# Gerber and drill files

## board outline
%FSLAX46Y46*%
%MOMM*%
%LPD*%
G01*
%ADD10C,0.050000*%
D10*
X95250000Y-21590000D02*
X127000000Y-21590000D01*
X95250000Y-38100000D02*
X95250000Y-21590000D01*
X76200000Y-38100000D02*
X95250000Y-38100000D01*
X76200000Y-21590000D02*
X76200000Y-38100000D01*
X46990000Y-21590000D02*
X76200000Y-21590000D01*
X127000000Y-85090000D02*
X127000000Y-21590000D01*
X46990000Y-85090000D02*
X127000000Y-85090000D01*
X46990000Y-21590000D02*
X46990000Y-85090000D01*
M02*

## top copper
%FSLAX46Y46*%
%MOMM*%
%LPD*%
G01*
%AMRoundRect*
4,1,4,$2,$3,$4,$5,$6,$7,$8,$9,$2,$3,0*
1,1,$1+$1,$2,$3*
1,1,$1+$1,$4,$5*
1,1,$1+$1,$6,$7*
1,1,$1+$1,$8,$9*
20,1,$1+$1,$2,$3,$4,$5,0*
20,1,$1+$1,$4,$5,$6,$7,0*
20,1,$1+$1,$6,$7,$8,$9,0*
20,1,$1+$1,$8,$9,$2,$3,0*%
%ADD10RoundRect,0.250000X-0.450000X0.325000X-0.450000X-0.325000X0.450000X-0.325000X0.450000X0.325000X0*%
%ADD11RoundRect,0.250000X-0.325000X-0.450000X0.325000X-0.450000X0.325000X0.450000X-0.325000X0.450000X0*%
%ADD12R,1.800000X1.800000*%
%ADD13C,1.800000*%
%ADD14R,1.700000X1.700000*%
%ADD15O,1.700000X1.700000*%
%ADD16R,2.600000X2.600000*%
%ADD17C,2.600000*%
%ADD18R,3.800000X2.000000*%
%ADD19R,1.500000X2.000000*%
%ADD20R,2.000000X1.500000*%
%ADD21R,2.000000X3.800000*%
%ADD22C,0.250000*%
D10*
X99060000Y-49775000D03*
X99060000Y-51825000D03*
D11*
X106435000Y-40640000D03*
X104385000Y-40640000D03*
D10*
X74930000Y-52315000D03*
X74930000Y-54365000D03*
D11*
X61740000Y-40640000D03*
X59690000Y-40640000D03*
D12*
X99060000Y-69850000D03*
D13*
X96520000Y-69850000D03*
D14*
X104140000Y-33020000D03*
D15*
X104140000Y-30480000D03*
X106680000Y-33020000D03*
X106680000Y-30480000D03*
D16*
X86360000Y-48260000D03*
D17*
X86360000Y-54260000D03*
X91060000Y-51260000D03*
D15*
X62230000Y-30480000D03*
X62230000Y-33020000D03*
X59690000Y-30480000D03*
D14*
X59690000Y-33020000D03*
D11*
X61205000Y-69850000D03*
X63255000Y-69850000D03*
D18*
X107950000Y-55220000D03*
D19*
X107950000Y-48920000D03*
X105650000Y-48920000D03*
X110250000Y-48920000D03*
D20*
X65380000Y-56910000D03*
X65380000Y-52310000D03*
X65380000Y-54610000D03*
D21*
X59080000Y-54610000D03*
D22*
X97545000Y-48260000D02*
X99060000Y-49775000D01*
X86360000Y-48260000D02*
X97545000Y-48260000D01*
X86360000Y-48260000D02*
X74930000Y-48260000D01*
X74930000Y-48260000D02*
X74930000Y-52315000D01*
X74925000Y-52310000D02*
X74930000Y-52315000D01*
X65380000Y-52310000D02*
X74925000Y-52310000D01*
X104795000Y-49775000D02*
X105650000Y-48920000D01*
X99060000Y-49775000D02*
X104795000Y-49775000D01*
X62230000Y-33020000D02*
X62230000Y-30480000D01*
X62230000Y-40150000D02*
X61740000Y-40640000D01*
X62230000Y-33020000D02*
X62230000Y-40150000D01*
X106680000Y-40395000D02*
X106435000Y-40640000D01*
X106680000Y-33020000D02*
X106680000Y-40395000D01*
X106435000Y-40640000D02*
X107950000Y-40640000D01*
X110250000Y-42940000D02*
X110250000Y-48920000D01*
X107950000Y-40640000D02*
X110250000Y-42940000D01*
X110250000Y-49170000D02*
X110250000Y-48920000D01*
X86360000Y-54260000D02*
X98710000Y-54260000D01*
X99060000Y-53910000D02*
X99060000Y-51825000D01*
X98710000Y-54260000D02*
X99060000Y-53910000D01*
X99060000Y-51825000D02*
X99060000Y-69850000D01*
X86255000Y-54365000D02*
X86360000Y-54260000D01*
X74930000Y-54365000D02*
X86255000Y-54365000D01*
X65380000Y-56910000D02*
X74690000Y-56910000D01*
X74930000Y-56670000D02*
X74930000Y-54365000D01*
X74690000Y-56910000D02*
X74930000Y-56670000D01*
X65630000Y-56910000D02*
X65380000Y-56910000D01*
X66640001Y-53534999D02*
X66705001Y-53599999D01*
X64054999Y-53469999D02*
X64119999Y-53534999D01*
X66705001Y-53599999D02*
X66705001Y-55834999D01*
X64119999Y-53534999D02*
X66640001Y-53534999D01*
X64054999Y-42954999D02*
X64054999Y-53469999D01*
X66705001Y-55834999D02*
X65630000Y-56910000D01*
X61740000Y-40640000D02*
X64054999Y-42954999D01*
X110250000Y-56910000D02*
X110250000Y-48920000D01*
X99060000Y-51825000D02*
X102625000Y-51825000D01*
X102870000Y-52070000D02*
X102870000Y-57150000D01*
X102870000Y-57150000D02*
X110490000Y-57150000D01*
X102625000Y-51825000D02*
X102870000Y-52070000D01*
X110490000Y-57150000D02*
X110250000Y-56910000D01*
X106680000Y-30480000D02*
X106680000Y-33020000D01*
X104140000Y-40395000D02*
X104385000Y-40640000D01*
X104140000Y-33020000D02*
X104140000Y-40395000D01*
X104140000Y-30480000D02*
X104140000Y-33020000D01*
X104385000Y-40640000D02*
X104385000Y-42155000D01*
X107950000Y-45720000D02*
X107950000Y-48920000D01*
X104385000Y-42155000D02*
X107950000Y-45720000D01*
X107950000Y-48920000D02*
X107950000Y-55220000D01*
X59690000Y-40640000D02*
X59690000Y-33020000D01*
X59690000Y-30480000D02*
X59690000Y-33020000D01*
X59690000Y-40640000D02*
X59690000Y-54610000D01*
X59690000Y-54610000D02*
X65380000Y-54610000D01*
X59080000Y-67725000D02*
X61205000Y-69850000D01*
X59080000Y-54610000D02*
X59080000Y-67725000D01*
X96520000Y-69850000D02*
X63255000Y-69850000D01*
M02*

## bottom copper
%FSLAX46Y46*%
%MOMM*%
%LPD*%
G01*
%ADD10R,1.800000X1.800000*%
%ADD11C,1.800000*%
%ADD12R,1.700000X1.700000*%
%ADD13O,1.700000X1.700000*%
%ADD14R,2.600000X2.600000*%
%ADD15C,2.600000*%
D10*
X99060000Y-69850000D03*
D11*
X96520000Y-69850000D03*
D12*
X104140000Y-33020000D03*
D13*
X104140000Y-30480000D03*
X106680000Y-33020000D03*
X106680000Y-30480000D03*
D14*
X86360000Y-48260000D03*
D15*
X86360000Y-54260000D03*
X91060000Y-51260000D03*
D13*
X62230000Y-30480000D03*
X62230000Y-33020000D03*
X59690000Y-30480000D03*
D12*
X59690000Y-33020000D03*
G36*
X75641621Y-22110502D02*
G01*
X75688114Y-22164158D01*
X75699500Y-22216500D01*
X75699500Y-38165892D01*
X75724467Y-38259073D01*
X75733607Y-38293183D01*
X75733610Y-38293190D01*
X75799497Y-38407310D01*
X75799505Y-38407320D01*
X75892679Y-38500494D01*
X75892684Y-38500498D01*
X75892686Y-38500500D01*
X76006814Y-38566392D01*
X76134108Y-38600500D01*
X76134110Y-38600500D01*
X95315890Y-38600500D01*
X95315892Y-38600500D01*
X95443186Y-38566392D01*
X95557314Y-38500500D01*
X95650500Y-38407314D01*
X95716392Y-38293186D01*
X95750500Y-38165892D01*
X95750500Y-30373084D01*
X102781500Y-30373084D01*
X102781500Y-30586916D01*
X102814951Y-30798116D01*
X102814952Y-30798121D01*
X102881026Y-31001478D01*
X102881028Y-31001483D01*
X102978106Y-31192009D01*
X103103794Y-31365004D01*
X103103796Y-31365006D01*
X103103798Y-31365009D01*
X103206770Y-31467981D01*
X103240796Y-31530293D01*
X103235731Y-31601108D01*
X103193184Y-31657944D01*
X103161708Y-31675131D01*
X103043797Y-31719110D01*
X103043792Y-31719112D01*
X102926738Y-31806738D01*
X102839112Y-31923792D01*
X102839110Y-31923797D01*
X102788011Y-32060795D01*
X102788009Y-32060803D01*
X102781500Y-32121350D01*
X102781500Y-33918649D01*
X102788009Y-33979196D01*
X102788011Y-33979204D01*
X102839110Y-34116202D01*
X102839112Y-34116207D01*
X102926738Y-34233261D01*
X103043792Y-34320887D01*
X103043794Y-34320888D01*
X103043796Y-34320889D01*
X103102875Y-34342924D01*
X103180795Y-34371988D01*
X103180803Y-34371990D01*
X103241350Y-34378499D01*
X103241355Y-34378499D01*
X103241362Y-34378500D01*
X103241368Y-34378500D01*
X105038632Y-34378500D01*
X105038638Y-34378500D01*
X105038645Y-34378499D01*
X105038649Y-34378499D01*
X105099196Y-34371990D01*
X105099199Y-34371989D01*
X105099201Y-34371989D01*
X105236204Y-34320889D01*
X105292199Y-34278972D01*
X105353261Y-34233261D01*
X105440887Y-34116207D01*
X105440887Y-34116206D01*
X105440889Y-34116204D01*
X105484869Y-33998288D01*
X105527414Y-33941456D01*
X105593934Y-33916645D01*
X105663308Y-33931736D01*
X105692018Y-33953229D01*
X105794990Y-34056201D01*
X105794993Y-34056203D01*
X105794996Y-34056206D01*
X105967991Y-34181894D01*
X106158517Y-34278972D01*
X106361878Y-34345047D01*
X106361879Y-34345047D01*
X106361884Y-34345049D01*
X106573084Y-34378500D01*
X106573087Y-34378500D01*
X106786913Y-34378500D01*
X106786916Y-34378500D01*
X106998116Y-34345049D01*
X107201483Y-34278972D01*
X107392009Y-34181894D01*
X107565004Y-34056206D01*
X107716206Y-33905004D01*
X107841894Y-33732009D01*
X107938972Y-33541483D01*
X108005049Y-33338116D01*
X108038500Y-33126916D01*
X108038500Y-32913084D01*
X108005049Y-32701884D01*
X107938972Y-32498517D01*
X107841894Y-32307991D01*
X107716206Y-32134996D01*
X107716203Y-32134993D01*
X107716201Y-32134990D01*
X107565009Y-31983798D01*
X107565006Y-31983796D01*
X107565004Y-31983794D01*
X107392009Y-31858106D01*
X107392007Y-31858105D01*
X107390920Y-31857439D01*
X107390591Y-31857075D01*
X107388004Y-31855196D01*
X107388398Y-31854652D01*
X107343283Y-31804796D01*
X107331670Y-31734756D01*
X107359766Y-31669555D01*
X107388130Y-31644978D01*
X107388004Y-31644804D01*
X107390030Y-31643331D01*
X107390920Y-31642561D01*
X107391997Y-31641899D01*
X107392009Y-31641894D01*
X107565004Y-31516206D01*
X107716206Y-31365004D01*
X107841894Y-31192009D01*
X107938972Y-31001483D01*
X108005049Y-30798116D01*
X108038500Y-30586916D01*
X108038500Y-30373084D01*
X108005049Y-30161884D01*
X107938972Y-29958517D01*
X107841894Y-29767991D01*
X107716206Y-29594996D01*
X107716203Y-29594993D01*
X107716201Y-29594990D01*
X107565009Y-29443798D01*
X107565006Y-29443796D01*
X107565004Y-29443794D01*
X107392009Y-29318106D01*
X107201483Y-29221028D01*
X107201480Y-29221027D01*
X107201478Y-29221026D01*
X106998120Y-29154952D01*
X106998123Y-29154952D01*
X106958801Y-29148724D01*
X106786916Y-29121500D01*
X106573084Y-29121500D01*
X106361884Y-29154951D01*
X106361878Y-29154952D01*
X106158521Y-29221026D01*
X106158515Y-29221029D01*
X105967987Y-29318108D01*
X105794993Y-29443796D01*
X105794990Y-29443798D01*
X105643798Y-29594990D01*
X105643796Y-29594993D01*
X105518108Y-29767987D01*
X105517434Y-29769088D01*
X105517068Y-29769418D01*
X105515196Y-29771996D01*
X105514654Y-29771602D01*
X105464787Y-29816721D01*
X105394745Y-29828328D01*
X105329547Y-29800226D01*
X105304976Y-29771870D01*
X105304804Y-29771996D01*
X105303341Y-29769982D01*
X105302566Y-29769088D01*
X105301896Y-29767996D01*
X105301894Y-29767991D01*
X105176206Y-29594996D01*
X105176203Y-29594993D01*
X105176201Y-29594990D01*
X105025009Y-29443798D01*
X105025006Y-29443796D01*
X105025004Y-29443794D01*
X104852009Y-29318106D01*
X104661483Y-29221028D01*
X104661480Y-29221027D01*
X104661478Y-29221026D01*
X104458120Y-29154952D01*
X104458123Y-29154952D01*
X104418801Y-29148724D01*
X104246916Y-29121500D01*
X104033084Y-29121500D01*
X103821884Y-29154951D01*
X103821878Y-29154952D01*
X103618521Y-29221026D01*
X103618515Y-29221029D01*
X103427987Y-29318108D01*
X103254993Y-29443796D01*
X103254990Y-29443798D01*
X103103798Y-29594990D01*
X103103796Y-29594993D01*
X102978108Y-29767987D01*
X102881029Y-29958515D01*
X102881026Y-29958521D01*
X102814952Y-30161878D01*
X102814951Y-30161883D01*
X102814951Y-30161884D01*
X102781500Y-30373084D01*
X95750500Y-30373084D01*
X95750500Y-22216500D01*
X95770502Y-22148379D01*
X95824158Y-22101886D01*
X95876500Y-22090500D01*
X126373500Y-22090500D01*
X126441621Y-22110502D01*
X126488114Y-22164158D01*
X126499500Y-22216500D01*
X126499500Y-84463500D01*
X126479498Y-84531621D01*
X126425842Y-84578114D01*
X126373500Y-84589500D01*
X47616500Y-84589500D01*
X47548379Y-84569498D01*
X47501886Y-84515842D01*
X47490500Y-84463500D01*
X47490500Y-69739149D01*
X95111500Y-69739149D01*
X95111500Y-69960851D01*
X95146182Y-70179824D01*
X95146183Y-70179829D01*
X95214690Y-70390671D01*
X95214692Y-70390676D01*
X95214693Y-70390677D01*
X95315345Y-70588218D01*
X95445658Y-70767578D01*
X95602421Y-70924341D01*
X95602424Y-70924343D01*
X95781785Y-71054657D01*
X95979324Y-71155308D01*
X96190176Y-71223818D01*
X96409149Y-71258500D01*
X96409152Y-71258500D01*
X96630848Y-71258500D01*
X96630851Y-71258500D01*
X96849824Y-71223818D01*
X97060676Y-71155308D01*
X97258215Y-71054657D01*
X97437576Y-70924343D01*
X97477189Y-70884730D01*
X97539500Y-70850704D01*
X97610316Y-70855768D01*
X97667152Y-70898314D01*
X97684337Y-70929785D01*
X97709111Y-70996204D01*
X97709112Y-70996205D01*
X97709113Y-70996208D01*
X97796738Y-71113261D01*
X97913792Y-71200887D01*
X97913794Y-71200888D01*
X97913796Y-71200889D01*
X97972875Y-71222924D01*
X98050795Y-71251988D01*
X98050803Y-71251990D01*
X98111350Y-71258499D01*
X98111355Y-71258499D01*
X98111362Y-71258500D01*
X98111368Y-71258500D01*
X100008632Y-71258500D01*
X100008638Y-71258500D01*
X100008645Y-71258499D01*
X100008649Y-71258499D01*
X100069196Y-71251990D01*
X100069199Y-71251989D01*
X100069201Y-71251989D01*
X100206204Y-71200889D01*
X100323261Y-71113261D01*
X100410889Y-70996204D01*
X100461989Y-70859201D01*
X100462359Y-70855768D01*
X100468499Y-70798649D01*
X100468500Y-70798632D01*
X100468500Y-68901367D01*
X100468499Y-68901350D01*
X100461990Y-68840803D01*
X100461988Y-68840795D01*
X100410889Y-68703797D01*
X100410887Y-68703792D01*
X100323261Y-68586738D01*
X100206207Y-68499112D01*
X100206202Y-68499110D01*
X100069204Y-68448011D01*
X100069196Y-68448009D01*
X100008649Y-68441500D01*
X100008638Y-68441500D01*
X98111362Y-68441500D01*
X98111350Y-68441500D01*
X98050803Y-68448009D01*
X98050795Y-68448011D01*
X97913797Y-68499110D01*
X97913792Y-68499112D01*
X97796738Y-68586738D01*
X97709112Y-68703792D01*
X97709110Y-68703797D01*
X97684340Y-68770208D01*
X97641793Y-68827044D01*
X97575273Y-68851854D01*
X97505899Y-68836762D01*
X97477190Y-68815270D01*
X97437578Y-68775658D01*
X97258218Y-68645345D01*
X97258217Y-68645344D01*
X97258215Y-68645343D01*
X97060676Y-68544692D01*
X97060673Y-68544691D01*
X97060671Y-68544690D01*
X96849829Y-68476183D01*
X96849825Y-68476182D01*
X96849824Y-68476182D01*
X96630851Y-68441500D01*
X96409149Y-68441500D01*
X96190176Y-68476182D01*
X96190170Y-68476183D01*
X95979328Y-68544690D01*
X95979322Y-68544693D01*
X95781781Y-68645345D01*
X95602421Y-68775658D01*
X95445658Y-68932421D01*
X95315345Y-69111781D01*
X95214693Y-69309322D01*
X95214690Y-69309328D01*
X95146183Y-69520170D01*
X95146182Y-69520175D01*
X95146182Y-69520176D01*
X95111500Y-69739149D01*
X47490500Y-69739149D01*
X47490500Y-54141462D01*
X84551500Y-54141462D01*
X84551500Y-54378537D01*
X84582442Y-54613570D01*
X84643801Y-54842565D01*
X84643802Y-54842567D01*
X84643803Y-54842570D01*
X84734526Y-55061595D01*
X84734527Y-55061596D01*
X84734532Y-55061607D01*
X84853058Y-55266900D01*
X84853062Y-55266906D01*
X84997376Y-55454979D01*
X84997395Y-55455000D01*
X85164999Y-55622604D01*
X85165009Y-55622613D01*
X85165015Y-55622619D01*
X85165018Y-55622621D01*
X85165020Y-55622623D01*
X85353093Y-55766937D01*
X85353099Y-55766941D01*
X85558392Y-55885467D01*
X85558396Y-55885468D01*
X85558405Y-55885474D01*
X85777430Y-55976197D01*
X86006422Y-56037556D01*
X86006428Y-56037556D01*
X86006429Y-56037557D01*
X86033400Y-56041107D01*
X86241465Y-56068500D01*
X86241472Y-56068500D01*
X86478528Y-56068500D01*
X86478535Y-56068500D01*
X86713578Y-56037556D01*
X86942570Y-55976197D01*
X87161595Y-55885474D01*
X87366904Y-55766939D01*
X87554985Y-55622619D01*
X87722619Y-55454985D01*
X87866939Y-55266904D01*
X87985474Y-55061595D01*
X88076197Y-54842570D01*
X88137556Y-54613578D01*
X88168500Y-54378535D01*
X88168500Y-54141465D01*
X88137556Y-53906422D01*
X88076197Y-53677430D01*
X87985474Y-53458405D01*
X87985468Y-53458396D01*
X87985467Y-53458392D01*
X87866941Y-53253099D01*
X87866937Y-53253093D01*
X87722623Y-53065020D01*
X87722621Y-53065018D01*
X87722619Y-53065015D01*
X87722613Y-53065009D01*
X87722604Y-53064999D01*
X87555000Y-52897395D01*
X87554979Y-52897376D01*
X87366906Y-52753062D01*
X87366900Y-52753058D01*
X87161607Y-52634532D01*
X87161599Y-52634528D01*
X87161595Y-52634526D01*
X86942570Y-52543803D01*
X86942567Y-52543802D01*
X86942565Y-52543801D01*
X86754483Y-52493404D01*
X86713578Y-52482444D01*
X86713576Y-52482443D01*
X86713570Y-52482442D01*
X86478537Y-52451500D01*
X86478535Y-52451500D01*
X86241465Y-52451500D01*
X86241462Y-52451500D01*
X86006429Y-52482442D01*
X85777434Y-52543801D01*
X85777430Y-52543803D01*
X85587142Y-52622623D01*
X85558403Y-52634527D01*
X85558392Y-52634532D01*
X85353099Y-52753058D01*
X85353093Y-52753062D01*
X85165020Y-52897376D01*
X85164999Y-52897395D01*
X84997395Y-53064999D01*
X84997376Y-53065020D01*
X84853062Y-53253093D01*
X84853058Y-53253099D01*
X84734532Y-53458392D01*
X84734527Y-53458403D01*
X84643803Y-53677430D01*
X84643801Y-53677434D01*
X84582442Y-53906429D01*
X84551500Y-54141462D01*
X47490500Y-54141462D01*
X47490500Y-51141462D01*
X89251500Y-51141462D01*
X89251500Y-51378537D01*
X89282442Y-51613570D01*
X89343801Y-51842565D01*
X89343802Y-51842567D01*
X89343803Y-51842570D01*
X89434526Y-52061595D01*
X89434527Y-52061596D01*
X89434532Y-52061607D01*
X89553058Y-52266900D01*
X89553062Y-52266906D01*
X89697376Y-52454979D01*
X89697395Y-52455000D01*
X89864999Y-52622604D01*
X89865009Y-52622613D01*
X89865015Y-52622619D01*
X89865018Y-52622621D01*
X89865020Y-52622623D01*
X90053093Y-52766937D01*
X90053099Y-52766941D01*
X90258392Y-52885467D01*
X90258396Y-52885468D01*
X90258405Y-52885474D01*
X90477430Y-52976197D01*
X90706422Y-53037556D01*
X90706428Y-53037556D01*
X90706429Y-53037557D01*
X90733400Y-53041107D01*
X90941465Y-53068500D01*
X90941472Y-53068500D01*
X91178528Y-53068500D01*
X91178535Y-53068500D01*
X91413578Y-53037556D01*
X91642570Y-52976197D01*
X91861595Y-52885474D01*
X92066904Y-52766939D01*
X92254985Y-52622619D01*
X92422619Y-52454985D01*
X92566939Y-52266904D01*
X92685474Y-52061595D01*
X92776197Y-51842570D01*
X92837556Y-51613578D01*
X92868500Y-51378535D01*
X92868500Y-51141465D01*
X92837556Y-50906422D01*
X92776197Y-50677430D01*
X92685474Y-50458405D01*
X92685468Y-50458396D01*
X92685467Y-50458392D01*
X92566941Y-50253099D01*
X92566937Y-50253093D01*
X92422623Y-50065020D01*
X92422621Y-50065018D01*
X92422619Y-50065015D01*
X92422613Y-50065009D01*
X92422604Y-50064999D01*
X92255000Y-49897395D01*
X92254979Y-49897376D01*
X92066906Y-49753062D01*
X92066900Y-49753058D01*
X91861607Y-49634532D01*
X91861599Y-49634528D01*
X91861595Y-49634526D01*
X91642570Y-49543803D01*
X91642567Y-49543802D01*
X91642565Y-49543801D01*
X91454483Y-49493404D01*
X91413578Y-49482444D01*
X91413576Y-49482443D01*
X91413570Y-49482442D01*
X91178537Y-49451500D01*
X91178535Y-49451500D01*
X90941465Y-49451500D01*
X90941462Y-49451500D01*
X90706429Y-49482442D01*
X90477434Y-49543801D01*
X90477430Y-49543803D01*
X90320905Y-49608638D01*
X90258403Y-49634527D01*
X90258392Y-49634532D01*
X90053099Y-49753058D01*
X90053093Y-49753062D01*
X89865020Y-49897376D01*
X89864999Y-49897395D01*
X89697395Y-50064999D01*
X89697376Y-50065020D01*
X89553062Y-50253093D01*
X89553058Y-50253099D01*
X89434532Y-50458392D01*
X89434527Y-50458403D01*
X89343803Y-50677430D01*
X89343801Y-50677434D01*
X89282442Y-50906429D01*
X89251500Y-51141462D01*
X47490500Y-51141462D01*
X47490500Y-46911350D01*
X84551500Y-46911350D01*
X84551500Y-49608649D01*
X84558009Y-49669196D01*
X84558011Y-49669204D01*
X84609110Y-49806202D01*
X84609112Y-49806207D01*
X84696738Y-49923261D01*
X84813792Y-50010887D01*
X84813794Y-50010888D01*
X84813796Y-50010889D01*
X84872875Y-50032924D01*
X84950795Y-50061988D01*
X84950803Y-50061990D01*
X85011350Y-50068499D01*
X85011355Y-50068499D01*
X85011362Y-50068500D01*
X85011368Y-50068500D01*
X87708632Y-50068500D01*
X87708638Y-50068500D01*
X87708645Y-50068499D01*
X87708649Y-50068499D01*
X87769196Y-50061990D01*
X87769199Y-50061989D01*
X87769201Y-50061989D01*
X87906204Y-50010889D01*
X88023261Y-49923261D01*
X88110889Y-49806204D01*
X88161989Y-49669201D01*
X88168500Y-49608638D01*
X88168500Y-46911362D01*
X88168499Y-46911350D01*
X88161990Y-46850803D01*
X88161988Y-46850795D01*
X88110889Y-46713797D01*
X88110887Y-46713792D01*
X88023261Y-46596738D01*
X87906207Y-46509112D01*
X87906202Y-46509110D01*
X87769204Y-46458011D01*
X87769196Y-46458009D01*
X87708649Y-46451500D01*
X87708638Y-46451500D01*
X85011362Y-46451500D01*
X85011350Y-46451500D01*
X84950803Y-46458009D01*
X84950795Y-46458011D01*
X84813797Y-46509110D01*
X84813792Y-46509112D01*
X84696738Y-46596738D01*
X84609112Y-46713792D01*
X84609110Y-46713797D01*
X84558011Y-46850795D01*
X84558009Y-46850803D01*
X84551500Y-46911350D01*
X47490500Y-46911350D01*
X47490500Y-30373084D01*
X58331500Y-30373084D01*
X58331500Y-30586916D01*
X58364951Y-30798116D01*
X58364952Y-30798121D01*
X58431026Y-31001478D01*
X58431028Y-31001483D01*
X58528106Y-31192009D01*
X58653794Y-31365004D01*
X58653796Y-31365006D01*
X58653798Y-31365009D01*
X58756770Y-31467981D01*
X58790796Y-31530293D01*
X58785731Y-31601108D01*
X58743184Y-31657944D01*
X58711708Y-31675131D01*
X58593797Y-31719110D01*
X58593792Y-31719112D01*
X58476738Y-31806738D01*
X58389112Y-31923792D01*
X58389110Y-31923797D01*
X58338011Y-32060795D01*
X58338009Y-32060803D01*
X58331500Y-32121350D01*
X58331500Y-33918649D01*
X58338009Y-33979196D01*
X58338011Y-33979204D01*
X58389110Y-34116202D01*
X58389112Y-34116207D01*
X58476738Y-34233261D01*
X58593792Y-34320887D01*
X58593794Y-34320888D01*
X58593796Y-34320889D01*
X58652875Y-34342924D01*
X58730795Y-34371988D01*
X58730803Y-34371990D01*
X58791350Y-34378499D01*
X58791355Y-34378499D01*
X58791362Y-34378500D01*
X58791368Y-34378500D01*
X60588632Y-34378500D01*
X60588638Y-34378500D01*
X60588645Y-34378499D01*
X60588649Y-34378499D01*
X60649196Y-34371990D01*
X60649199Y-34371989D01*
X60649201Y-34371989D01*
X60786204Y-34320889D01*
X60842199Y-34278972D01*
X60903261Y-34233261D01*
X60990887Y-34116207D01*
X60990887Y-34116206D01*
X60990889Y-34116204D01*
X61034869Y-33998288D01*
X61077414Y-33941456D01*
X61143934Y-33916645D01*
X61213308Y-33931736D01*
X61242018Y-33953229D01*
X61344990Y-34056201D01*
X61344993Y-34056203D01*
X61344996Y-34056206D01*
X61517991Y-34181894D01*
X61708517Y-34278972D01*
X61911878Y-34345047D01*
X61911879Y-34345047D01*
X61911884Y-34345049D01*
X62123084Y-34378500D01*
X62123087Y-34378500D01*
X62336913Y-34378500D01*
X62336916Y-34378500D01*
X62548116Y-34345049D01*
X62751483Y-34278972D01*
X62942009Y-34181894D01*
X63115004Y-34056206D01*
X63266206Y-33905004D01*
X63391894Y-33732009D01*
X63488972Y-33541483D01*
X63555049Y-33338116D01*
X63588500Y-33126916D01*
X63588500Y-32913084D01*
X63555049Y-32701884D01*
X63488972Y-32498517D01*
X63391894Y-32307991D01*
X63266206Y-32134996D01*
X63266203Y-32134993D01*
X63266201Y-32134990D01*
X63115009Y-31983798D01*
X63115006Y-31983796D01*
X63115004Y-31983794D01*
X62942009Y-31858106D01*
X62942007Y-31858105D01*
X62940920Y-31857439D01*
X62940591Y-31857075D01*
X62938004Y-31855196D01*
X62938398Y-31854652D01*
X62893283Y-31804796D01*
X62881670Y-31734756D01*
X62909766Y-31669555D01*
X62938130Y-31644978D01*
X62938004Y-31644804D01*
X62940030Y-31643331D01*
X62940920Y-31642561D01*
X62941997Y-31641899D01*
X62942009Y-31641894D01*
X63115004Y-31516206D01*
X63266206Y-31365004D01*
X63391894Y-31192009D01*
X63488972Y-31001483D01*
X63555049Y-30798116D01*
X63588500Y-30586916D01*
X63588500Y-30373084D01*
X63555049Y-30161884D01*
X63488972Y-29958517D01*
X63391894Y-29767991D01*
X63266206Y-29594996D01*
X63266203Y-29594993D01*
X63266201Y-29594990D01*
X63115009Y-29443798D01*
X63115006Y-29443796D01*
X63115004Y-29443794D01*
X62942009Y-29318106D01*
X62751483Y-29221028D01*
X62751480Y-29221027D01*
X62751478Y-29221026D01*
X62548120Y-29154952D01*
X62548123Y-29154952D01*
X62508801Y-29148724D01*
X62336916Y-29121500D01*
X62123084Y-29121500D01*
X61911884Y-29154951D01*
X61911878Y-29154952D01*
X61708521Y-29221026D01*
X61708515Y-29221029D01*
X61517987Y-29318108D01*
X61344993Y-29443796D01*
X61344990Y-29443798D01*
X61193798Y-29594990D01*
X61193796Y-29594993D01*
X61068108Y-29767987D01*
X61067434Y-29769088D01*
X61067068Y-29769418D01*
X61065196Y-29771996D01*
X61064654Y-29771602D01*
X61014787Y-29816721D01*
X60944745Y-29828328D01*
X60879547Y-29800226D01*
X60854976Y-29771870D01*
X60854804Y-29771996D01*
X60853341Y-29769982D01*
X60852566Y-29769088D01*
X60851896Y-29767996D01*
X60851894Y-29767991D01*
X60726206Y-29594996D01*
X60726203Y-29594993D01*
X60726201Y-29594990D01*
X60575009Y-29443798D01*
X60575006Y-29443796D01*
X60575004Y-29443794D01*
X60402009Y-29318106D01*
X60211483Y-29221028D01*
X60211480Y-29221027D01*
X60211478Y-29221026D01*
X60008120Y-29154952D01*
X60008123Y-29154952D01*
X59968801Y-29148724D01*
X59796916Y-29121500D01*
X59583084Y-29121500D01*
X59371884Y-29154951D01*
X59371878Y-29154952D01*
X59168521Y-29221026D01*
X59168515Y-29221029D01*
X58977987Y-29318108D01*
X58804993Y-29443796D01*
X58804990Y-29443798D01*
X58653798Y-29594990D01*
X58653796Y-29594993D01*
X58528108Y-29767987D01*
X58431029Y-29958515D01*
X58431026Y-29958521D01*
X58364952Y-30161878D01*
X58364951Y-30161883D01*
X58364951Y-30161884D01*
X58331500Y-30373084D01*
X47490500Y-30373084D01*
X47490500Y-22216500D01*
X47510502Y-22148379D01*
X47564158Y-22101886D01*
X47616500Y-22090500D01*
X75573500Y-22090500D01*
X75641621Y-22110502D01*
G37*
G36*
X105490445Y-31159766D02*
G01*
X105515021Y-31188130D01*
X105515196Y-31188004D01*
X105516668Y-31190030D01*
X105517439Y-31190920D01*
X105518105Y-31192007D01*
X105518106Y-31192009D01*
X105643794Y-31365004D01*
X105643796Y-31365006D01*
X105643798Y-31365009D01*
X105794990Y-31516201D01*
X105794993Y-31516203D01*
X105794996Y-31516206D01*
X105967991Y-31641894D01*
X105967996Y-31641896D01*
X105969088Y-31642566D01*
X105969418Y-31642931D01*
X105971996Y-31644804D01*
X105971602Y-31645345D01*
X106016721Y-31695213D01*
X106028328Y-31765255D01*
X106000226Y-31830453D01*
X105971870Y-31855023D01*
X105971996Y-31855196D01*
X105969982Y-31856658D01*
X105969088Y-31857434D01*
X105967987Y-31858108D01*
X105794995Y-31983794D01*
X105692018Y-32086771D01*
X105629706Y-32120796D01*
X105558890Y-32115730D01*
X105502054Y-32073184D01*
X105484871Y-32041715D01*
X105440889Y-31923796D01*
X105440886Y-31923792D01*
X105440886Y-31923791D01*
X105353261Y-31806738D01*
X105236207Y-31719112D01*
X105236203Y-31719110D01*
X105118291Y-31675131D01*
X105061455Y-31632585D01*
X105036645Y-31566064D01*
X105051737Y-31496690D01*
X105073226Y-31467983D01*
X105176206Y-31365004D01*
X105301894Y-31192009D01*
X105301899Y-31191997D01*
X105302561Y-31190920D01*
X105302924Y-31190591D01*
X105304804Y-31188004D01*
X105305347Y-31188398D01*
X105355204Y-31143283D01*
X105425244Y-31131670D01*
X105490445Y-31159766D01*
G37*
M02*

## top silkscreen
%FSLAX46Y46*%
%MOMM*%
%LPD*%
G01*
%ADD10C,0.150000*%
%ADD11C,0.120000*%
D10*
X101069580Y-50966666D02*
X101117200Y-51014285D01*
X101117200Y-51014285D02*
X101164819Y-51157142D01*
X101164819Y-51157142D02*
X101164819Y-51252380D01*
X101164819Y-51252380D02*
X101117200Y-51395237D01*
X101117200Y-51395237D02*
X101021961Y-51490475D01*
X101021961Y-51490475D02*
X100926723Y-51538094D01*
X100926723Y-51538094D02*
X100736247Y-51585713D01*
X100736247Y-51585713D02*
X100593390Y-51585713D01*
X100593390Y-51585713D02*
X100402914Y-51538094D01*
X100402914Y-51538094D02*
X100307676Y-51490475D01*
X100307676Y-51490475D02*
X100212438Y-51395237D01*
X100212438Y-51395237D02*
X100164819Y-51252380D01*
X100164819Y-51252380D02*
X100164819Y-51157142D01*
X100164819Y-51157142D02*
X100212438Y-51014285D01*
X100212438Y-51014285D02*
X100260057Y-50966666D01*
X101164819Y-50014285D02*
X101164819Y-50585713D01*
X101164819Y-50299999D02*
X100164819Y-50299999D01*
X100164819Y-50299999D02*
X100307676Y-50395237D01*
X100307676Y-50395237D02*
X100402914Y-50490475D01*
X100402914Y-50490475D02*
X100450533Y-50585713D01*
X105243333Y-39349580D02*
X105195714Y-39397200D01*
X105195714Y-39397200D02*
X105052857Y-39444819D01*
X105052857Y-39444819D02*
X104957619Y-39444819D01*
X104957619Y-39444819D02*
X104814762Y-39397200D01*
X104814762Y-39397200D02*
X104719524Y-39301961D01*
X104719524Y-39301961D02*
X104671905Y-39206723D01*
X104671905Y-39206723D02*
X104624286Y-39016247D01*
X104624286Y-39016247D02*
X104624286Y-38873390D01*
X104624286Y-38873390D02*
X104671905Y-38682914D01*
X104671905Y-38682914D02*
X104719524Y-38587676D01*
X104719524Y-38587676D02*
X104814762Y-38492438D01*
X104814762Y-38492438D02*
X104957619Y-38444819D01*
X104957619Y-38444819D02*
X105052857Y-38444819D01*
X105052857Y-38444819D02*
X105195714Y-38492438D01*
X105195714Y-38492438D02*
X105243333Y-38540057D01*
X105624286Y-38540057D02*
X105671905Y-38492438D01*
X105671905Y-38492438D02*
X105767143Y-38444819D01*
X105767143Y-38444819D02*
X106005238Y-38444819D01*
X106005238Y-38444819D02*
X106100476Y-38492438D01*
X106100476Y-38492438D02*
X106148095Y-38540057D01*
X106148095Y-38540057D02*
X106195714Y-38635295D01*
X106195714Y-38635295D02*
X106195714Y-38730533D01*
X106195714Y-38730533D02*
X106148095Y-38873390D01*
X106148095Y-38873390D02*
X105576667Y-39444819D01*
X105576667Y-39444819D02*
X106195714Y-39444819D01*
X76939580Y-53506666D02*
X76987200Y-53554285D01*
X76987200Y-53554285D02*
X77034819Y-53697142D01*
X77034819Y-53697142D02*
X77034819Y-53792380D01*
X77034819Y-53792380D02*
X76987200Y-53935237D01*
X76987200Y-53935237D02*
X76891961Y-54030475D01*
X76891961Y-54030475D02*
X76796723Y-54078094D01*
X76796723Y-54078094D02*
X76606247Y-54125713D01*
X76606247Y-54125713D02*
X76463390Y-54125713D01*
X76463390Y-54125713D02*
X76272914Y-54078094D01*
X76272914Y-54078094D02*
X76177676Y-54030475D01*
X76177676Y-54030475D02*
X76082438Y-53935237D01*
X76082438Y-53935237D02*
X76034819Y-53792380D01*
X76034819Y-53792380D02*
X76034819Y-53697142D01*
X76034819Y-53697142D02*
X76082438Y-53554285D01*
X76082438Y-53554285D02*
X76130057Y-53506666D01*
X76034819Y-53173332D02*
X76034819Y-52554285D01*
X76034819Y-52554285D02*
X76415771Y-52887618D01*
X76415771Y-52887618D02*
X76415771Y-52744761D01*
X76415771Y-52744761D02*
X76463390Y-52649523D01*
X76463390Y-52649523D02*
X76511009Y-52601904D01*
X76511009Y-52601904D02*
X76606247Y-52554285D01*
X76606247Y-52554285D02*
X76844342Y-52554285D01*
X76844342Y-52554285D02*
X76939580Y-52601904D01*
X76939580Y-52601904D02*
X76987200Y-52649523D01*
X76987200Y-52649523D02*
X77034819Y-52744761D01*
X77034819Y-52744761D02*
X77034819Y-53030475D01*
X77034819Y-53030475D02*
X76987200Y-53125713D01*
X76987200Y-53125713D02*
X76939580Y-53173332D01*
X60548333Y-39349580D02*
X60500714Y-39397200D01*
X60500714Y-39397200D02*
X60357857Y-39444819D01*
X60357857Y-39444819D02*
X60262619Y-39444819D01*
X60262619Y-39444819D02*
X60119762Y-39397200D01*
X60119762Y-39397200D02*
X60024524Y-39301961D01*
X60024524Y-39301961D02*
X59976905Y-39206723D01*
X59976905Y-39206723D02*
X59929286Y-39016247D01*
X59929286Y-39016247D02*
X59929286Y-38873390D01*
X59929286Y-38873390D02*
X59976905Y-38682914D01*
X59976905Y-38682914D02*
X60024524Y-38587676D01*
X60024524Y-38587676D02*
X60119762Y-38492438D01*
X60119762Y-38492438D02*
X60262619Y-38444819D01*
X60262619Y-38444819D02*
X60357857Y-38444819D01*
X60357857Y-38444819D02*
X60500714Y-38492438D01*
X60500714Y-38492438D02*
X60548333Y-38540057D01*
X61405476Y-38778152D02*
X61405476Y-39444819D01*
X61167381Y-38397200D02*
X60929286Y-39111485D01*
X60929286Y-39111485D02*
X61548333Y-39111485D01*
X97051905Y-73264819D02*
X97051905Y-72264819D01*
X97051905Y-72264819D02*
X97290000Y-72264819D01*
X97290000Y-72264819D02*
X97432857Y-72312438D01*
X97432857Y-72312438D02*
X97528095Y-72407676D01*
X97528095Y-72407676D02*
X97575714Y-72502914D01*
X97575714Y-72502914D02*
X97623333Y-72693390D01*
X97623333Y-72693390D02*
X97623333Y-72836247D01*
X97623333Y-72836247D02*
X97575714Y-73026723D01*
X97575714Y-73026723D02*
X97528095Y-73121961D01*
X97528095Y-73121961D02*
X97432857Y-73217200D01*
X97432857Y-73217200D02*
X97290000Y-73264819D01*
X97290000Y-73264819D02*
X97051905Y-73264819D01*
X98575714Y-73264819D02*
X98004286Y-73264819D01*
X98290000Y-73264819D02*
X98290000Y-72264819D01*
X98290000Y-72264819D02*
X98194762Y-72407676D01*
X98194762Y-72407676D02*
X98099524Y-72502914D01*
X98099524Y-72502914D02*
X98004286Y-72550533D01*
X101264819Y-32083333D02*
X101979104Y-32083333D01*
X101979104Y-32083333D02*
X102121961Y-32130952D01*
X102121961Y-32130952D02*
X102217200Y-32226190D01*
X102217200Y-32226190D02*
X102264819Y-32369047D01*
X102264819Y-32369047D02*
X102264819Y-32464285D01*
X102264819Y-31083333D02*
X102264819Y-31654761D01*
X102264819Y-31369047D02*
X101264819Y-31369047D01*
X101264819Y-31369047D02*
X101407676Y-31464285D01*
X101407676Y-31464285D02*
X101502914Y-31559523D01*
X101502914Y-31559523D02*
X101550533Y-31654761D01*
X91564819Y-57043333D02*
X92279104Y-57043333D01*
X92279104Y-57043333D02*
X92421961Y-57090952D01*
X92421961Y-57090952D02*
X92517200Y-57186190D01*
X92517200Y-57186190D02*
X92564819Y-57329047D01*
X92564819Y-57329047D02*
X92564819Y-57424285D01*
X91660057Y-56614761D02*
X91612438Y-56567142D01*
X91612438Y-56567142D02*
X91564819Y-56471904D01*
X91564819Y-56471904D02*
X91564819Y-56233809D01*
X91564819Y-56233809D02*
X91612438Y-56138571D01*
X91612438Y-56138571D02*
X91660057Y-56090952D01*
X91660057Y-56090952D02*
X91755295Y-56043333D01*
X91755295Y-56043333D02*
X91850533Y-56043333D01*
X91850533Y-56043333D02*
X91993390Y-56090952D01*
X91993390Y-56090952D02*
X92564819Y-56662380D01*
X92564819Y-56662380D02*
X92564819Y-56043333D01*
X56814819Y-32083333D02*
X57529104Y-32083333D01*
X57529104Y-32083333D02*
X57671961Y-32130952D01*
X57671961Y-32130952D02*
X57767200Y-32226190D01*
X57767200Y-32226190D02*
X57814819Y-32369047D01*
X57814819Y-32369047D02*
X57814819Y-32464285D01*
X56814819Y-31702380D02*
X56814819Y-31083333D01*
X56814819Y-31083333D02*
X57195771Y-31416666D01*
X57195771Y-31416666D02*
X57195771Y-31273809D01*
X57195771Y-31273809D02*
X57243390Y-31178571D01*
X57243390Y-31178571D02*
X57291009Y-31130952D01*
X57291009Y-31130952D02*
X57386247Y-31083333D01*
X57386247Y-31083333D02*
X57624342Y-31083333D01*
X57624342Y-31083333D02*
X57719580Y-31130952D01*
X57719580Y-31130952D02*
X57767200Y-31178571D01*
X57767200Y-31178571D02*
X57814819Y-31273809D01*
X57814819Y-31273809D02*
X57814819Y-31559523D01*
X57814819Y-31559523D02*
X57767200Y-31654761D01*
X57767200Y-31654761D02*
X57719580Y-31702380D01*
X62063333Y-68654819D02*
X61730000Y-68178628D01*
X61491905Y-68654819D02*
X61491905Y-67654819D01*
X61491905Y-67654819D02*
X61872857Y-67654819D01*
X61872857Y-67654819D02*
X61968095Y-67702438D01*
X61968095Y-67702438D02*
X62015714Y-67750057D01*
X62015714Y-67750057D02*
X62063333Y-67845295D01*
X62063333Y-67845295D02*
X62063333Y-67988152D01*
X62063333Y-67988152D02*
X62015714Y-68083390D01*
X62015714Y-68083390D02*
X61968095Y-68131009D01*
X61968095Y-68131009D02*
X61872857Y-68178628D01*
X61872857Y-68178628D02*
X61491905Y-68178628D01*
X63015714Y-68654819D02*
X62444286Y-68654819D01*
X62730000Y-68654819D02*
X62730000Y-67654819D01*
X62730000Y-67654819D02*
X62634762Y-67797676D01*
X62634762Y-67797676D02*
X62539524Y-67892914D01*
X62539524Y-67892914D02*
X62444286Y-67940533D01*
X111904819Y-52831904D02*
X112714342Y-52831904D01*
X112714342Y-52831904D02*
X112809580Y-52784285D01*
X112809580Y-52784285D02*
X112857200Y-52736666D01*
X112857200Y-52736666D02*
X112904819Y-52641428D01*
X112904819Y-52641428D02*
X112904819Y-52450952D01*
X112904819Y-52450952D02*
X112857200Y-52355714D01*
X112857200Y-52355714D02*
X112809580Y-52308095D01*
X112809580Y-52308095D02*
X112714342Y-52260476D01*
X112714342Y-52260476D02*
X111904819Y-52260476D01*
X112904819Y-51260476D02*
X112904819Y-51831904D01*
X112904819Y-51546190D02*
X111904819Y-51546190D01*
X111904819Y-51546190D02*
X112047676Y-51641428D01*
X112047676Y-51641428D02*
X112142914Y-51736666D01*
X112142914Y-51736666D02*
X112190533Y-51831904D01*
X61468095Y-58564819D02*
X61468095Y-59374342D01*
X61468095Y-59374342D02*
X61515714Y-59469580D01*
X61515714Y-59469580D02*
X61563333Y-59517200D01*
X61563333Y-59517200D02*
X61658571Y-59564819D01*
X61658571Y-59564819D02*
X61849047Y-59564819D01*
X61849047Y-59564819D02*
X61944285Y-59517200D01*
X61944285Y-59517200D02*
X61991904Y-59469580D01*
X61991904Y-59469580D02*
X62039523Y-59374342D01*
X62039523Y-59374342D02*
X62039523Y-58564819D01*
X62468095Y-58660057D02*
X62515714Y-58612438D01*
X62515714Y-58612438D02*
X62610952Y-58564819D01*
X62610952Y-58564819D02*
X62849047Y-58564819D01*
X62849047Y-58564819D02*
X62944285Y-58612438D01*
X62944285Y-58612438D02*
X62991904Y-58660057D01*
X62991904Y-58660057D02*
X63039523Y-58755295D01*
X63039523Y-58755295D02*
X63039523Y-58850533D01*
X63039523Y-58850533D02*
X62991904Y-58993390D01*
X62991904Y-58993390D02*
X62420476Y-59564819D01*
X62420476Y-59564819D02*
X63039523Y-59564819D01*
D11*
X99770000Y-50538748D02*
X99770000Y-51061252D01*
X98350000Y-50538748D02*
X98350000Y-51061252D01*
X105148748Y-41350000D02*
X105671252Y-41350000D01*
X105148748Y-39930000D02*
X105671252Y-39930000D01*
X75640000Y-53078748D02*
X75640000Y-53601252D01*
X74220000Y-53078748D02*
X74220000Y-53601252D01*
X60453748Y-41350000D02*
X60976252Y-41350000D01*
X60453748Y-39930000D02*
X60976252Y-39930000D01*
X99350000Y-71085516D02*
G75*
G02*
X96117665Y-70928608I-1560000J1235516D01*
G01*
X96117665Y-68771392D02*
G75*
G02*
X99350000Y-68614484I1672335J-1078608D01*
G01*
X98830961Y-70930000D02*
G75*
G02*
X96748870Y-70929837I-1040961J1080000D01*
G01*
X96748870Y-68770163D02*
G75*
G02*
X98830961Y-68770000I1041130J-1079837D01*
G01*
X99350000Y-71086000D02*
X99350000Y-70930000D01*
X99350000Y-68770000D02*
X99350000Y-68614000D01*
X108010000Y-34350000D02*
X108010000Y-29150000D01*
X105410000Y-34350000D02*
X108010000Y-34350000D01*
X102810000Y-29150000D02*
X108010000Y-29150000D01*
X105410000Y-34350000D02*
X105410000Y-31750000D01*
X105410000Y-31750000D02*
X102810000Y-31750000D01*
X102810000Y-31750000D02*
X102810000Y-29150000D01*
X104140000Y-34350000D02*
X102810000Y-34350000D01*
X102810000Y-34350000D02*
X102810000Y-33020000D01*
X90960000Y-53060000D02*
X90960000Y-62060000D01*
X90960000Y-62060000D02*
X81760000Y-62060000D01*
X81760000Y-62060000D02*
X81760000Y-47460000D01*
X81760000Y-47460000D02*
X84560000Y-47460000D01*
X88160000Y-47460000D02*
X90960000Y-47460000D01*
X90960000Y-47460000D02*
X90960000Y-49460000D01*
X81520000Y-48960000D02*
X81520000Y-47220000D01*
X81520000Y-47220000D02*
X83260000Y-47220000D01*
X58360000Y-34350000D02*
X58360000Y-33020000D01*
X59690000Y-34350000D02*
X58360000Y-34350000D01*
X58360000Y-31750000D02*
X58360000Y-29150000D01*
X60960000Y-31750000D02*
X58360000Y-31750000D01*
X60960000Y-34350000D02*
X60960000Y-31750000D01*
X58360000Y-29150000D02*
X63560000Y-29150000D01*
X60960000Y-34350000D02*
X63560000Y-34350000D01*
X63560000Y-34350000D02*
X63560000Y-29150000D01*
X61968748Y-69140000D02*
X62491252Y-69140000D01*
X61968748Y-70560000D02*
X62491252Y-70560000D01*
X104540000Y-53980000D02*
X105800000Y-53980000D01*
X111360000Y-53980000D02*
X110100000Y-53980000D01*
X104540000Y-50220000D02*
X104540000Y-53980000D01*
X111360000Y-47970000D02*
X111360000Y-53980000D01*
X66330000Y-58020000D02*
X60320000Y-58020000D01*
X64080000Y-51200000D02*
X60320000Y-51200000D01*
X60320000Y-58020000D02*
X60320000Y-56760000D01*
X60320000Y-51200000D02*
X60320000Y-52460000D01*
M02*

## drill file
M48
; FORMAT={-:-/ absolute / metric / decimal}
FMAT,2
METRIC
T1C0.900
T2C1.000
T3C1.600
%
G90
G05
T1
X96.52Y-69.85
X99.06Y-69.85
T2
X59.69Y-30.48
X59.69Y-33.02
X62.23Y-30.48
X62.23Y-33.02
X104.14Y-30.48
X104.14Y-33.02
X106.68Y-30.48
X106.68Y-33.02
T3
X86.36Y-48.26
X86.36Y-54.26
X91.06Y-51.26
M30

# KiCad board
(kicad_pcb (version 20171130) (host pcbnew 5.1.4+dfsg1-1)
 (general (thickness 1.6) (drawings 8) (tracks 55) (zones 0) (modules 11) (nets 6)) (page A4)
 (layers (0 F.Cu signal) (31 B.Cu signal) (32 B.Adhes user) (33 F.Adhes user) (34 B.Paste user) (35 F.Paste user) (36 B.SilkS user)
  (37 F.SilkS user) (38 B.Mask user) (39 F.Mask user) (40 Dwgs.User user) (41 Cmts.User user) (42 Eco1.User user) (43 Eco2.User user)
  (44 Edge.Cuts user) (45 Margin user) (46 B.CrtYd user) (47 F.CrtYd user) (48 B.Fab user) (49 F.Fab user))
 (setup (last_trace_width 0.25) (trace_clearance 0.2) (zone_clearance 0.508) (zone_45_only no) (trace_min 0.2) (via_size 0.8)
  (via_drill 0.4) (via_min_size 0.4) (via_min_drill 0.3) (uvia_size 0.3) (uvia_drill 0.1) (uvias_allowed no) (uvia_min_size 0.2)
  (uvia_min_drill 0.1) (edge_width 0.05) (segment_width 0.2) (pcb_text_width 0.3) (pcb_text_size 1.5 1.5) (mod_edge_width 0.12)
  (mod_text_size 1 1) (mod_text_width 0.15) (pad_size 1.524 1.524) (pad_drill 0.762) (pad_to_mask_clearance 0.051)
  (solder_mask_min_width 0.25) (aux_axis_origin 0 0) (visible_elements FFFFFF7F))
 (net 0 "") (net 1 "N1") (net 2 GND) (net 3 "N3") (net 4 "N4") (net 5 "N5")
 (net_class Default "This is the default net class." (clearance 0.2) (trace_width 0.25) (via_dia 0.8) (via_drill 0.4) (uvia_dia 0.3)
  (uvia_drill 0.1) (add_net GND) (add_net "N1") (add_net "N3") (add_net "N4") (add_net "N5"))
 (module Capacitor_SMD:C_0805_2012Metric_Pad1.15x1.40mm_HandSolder (layer F.Cu) (at 99.06 50.8 270)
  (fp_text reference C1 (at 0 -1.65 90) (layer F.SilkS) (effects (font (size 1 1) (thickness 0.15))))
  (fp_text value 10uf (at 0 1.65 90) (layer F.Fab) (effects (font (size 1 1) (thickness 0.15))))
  (fp_line (start -0.261252 -0.71) (end 0.261252 -0.71) (layer F.SilkS) (width 0.12))
  (fp_line (start -0.261252 0.71) (end 0.261252 0.71) (layer F.SilkS) (width 0.12))
  (pad 1 smd roundrect (at -1.025 0 270) (size 1.15 1.4) (layers F.Cu F.Paste F.Mask) (roundrect_rratio 0.217391) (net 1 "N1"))
  (pad 2 smd roundrect (at 1.025 0 270) (size 1.15 1.4) (layers F.Cu F.Paste F.Mask) (roundrect_rratio 0.217391) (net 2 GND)))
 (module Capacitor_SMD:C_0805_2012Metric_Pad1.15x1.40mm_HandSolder (layer F.Cu) (at 105.41 40.64)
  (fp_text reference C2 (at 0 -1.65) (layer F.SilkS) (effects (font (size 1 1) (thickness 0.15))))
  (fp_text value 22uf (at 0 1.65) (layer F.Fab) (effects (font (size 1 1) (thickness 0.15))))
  (fp_line (start -0.261252 0.71) (end 0.261252 0.71) (layer F.SilkS) (width 0.12))
  (fp_line (start -0.261252 -0.71) (end 0.261252 -0.71) (layer F.SilkS) (width 0.12))
  (pad 2 smd roundrect (at 1.025 0) (size 1.15 1.4) (layers F.Cu F.Paste F.Mask) (roundrect_rratio 0.217391) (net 2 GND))
  (pad 1 smd roundrect (at -1.025 0) (size 1.15 1.4) (layers F.Cu F.Paste F.Mask) (roundrect_rratio 0.217391) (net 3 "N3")))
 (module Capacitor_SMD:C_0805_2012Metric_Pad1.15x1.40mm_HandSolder (layer F.Cu) (at 74.93 53.34 270)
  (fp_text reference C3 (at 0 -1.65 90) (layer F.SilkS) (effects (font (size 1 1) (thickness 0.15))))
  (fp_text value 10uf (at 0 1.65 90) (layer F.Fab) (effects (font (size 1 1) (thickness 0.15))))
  (fp_line (start -0.261252 -0.71) (end 0.261252 -0.71) (layer F.SilkS) (width 0.12))
  (fp_line (start -0.261252 0.71) (end 0.261252 0.71) (layer F.SilkS) (width 0.12))
  (pad 1 smd roundrect (at -1.025 0 270) (size 1.15 1.4) (layers F.Cu F.Paste F.Mask) (roundrect_rratio 0.217391) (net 1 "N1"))
  (pad 2 smd roundrect (at 1.025 0 270) (size 1.15 1.4) (layers F.Cu F.Paste F.Mask) (roundrect_rratio 0.217391) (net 2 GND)))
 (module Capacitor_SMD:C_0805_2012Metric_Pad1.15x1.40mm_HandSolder (layer F.Cu) (at 60.715 40.64)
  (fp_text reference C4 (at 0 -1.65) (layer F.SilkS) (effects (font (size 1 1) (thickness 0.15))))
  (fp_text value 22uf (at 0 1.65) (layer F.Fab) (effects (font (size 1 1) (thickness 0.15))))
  (fp_line (start -0.261252 0.71) (end 0.261252 0.71) (layer F.SilkS) (width 0.12))
  (fp_line (start -0.261252 -0.71) (end 0.261252 -0.71) (layer F.SilkS) (width 0.12))
  (pad 2 smd roundrect (at 1.025 0) (size 1.15 1.4) (layers F.Cu F.Paste F.Mask) (roundrect_rratio 0.217391) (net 2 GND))
  (pad 1 smd roundrect (at -1.025 0) (size 1.15 1.4) (layers F.Cu F.Paste F.Mask) (roundrect_rratio 0.217391) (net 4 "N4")))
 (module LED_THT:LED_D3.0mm (layer F.Cu) (at 99.06 69.85 180)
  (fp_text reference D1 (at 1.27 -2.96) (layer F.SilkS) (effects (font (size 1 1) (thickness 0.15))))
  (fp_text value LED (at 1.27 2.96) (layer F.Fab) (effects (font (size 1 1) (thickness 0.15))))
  (fp_arc (start 1.27 0) (end -0.29 -1.235516) (angle 108.8) (layer F.SilkS) (width 0.12))
  (fp_arc (start 1.27 0) (end -0.29 1.235516) (angle -108.8) (layer F.SilkS) (width 0.12))
  (fp_arc (start 1.27 0) (end 0.229039 -1.08) (angle 87.9) (layer F.SilkS) (width 0.12))
  (fp_arc (start 1.27 0) (end 0.229039 1.08) (angle -87.9) (layer F.SilkS) (width 0.12))
  (fp_line (start -0.29 -1.236) (end -0.29 -1.08) (layer F.SilkS) (width 0.12))
  (fp_line (start -0.29 1.08) (end -0.29 1.236) (layer F.SilkS) (width 0.12))
  (pad 1 thru_hole rect (at 0 0 180) (size 1.8 1.8) (drill 0.9) (layers *.Cu *.Mask) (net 2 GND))
  (pad 2 thru_hole circle (at 2.54 0 180) (size 1.8 1.8) (drill 0.9) (layers *.Cu *.Mask) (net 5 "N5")))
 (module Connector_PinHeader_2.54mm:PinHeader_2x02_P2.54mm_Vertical (layer F.Cu) (at 104.14 33.02 90)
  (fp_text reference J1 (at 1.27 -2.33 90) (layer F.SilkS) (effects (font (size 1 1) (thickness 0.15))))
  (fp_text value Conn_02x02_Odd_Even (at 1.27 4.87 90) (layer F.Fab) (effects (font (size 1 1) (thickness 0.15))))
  (fp_line (start -1.33 3.87) (end 3.87 3.87) (layer F.SilkS) (width 0.12))
  (fp_line (start -1.33 1.27) (end -1.33 3.87) (layer F.SilkS) (width 0.12))
  (fp_line (start 3.87 -1.33) (end 3.87 3.87) (layer F.SilkS) (width 0.12))
  (fp_line (start -1.33 1.27) (end 1.27 1.27) (layer F.SilkS) (width 0.12))
  (fp_line (start 1.27 1.27) (end 1.27 -1.33) (layer F.SilkS) (width 0.12))
  (fp_line (start 1.27 -1.33) (end 3.87 -1.33) (layer F.SilkS) (width 0.12))
  (fp_line (start -1.33 0) (end -1.33 -1.33) (layer F.SilkS) (width 0.12))
  (fp_line (start -1.33 -1.33) (end 0 -1.33) (layer F.SilkS) (width 0.12))
  (pad 1 thru_hole rect (at 0 0 90) (size 1.7 1.7) (drill 1) (layers *.Cu *.Mask) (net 3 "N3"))
  (pad 2 thru_hole oval (at 2.54 0 90) (size 1.7 1.7) (drill 1) (layers *.Cu *.Mask) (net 3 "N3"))
  (pad 3 thru_hole oval (at 0 2.54 90) (size 1.7 1.7) (drill 1) (layers *.Cu *.Mask) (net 2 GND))
  (pad 4 thru_hole oval (at 2.54 2.54 90) (size 1.7 1.7) (drill 1) (layers *.Cu *.Mask) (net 2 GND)))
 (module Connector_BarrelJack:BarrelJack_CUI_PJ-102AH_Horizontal (layer F.Cu) (at 86.36 48.26)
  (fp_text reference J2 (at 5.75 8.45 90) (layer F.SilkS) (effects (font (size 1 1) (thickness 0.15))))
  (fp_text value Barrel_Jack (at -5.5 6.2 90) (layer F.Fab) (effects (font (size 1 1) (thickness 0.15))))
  (fp_line (start 4.6 4.8) (end 4.6 13.8) (layer F.SilkS) (width 0.12))
  (fp_line (start 4.6 13.8) (end -4.6 13.8) (layer F.SilkS) (width 0.12))
  (fp_line (start -4.6 13.8) (end -4.6 -0.8) (layer F.SilkS) (width 0.12))
  (fp_line (start -4.6 -0.8) (end -1.8 -0.8) (layer F.SilkS) (width 0.12))
  (fp_line (start 1.8 -0.8) (end 4.6 -0.8) (layer F.SilkS) (width 0.12))
  (fp_line (start 4.6 -0.8) (end 4.6 1.2) (layer F.SilkS) (width 0.12))
  (fp_line (start -4.84 0.7) (end -4.84 -1.04) (layer F.SilkS) (width 0.12))
  (fp_line (start -4.84 -1.04) (end -3.1 -1.04) (layer F.SilkS) (width 0.12))
  (pad 1 thru_hole rect (at 0 0) (size 2.6 2.6) (drill 1.6) (layers *.Cu *.Mask) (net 1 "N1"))
  (pad 2 thru_hole circle (at 0 6) (size 2.6 2.6) (drill 1.6) (layers *.Cu *.Mask) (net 2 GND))
  (pad 3 thru_hole circle (at 4.7 3) (size 2.6 2.6) (drill 1.6) (layers *.Cu *.Mask)))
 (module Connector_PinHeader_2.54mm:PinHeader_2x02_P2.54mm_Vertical (layer F.Cu) (at 59.69 33.02 90)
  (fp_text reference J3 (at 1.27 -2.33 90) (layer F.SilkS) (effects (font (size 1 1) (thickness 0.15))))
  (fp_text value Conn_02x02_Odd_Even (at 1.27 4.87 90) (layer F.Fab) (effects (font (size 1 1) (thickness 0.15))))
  (fp_line (start -1.33 -1.33) (end 0 -1.33) (layer F.SilkS) (width 0.12))
  (fp_line (start -1.33 0) (end -1.33 -1.33) (layer F.SilkS) (width 0.12))
  (fp_line (start 1.27 -1.33) (end 3.87 -1.33) (layer F.SilkS) (width 0.12))
  (fp_line (start 1.27 1.27) (end 1.27 -1.33) (layer F.SilkS) (width 0.12))
  (fp_line (start -1.33 1.27) (end 1.27 1.27) (layer F.SilkS) (width 0.12))
  (fp_line (start 3.87 -1.33) (end 3.87 3.87) (layer F.SilkS) (width 0.12))
  (fp_line (start -1.33 1.27) (end -1.33 3.87) (layer F.SilkS) (width 0.12))
  (fp_line (start -1.33 3.87) (end 3.87 3.87) (layer F.SilkS) (width 0.12))
  (pad 4 thru_hole oval (at 2.54 2.54 90) (size 1.7 1.7) (drill 1) (layers *.Cu *.Mask) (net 2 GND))
  (pad 3 thru_hole oval (at 0 2.54 90) (size 1.7 1.7) (drill 1) (layers *.Cu *.Mask) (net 2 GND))
  (pad 2 thru_hole oval (at 2.54 0 90) (size 1.7 1.7) (drill 1) (layers *.Cu *.Mask) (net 4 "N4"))
  (pad 1 thru_hole rect (at 0 0 90) (size 1.7 1.7) (drill 1) (layers *.Cu *.Mask) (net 4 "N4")))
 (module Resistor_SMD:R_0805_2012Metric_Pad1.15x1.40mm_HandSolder (layer F.Cu) (at 62.23 69.85)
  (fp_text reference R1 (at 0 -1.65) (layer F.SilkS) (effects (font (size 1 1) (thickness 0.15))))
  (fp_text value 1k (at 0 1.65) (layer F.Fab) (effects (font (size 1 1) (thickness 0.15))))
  (fp_line (start -0.261252 -0.71) (end 0.261252 -0.71) (layer F.SilkS) (width 0.12))
  (fp_line (start -0.261252 0.71) (end 0.261252 0.71) (layer F.SilkS) (width 0.12))
  (pad 1 smd roundrect (at -1.025 0) (size 1.15 1.4) (layers F.Cu F.Paste F.Mask) (roundrect_rratio 0.217391) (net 4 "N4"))
  (pad 2 smd roundrect (at 1.025 0) (size 1.15 1.4) (layers F.Cu F.Paste F.Mask) (roundrect_rratio 0.217391) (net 5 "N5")))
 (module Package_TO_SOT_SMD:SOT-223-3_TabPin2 (layer F.Cu) (at 107.95 52.07 270)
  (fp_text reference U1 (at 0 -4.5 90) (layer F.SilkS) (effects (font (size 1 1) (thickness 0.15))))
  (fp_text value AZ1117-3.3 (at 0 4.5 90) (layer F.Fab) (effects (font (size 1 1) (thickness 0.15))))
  (fp_line (start 1.91 3.41) (end 1.91 2.15) (layer F.SilkS) (width 0.12))
  (fp_line (start 1.91 -3.41) (end 1.91 -2.15) (layer F.SilkS) (width 0.12))
  (fp_line (start -1.85 3.41) (end 1.91 3.41) (layer F.SilkS) (width 0.12))
  (fp_line (start -4.1 -3.41) (end 1.91 -3.41) (layer F.SilkS) (width 0.12))
  (pad 2 smd rect (at 3.15 0 270) (size 2 3.8) (layers F.Cu F.Paste F.Mask) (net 3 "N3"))
  (pad 2 smd rect (at -3.15 0 270) (size 2 1.5) (layers F.Cu F.Paste F.Mask) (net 3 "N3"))
  (pad 3 smd rect (at -3.15 2.3 270) (size 2 1.5) (layers F.Cu F.Paste F.Mask) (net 1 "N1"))
  (pad 1 smd rect (at -3.15 -2.3 270) (size 2 1.5) (layers F.Cu F.Paste F.Mask) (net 2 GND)))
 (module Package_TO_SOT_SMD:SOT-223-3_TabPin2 (layer F.Cu) (at 62.23 54.61 180)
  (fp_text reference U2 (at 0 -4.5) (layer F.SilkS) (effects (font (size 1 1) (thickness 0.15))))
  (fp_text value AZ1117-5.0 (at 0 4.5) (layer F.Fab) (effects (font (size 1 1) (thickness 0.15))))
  (fp_line (start -4.1 -3.41) (end 1.91 -3.41) (layer F.SilkS) (width 0.12))
  (fp_line (start -1.85 3.41) (end 1.91 3.41) (layer F.SilkS) (width 0.12))
  (fp_line (start 1.91 -3.41) (end 1.91 -2.15) (layer F.SilkS) (width 0.12))
  (fp_line (start 1.91 3.41) (end 1.91 2.15) (layer F.SilkS) (width 0.12))
  (pad 1 smd rect (at -3.15 -2.3 180) (size 2 1.5) (layers F.Cu F.Paste F.Mask) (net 2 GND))
  (pad 3 smd rect (at -3.15 2.3 180) (size 2 1.5) (layers F.Cu F.Paste F.Mask) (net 1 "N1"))
  (pad 2 smd rect (at -3.15 0 180) (size 2 1.5) (layers F.Cu F.Paste F.Mask) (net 4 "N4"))
  (pad 2 smd rect (at 3.15 0 180) (size 2 3.8) (layers F.Cu F.Paste F.Mask) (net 4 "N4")))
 (gr_line (start 95.25 21.59) (end 127 21.59) (layer Edge.Cuts) (width 0.05))
 (gr_line (start 95.25 38.1) (end 95.25 21.59) (layer Edge.Cuts) (width 0.05))
 (gr_line (start 76.2 38.1) (end 95.25 38.1) (layer Edge.Cuts) (width 0.05))
 (gr_line (start 76.2 21.59) (end 76.2 38.1) (layer Edge.Cuts) (width 0.05))
 (gr_line (start 46.99 21.59) (end 76.2 21.59) (layer Edge.Cuts) (width 0.05))
 (gr_line (start 127 85.09) (end 127 21.59) (layer Edge.Cuts) (width 0.05))
 (gr_line (start 46.99 85.09) (end 127 85.09) (layer Edge.Cuts) (width 0.05))
 (gr_line (start 46.99 21.59) (end 46.99 85.09) (layer Edge.Cuts) (width 0.05))
 (segment (start 97.545 48.26) (end 99.06 49.775) (width 0.25) (layer F.Cu) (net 1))
 (segment (start 86.36 48.26) (end 97.545 48.26) (width 0.25) (layer F.Cu) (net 1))
 (segment (start 86.36 48.26) (end 74.93 48.26) (width 0.25) (layer F.Cu) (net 1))
 (segment (start 74.93 48.26) (end 74.93 52.315) (width 0.25) (layer F.Cu) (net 1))
 (segment (start 74.925 52.31) (end 74.93 52.315) (width 0.25) (layer F.Cu) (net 1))
 (segment (start 65.38 52.31) (end 74.925 52.31) (width 0.25) (layer F.Cu) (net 1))
 (segment (start 104.795 49.775) (end 105.65 48.92) (width 0.25) (layer F.Cu) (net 1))
 (segment (start 99.06 49.775) (end 104.795 49.775) (width 0.25) (layer F.Cu) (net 1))
 (segment (start 62.23 33.02) (end 62.23 30.48) (width 0.25) (layer F.Cu) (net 2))
 (segment (start 62.23 40.15) (end 61.74 40.64) (width 0.25) (layer F.Cu) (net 2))
 (segment (start 62.23 33.02) (end 62.23 40.15) (width 0.25) (layer F.Cu) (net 2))
 (segment (start 106.68 40.395) (end 106.435 40.64) (width 0.25) (layer F.Cu) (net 2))
 (segment (start 106.68 33.02) (end 106.68 40.395) (width 0.25) (layer F.Cu) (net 2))
 (segment (start 106.435 40.64) (end 107.95 40.64) (width 0.25) (layer F.Cu) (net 2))
 (segment (start 110.25 42.94) (end 110.25 48.92) (width 0.25) (layer F.Cu) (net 2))
 (segment (start 107.95 40.64) (end 110.25 42.94) (width 0.25) (layer F.Cu) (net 2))
 (segment (start 110.25 49.17) (end 110.25 48.92) (width 0.25) (layer F.Cu) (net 2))
 (segment (start 86.36 54.26) (end 98.71 54.26) (width 0.25) (layer F.Cu) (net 2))
 (segment (start 99.06 53.91) (end 99.06 51.825) (width 0.25) (layer F.Cu) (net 2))
 (segment (start 98.71 54.26) (end 99.06 53.91) (width 0.25) (layer F.Cu) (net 2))
 (segment (start 99.06 51.825) (end 99.06 69.85) (width 0.25) (layer F.Cu) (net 2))
 (segment (start 86.255 54.365) (end 86.36 54.26) (width 0.25) (layer F.Cu) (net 2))
 (segment (start 74.93 54.365) (end 86.255 54.365) (width 0.25) (layer F.Cu) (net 2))
 (segment (start 65.38 56.91) (end 74.69 56.91) (width 0.25) (layer F.Cu) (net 2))
 (segment (start 74.93 56.67) (end 74.93 54.365) (width 0.25) (layer F.Cu) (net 2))
 (segment (start 74.69 56.91) (end 74.93 56.67) (width 0.25) (layer F.Cu) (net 2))
 (segment (start 65.63 56.91) (end 65.38 56.91) (width 0.25) (layer F.Cu) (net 2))
 (segment (start 66.640001 53.534999) (end 66.705001 53.599999) (width 0.25) (layer F.Cu) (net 2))
 (segment (start 64.054999 53.469999) (end 64.119999 53.534999) (width 0.25) (layer F.Cu) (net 2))
 (segment (start 66.705001 53.599999) (end 66.705001 55.834999) (width 0.25) (layer F.Cu) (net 2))
 (segment (start 64.119999 53.534999) (end 66.640001 53.534999) (width 0.25) (layer F.Cu) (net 2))
 (segment (start 64.054999 42.954999) (end 64.054999 53.469999) (width 0.25) (layer F.Cu) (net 2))
 (segment (start 66.705001 55.834999) (end 65.63 56.91) (width 0.25) (layer F.Cu) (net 2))
 (segment (start 61.74 40.64) (end 64.054999 42.954999) (width 0.25) (layer F.Cu) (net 2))
 (segment (start 110.25 56.91) (end 110.25 48.92) (width 0.25) (layer F.Cu) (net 2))
 (segment (start 99.06 51.825) (end 102.625 51.825) (width 0.25) (layer F.Cu) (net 2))
 (segment (start 102.87 52.07) (end 102.87 57.15) (width 0.25) (layer F.Cu) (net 2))
 (segment (start 102.87 57.15) (end 110.49 57.15) (width 0.25) (layer F.Cu) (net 2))
 (segment (start 102.625 51.825) (end 102.87 52.07) (width 0.25) (layer F.Cu) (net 2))
 (segment (start 110.49 57.15) (end 110.25 56.91) (width 0.25) (layer F.Cu) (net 2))
 (segment (start 106.68 30.48) (end 106.68 33.02) (width 0.25) (layer F.Cu) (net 2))
 (segment (start 104.14 40.395) (end 104.385 40.64) (width 0.25) (layer F.Cu) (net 3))
 (segment (start 104.14 33.02) (end 104.14 40.395) (width 0.25) (layer F.Cu) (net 3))
 (segment (start 104.14 30.48) (end 104.14 33.02) (width 0.25) (layer F.Cu) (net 3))
 (segment (start 104.385 40.64) (end 104.385 42.155) (width 0.25) (layer F.Cu) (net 3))
 (segment (start 107.95 45.72) (end 107.95 48.92) (width 0.25) (layer F.Cu) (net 3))
 (segment (start 104.385 42.155) (end 107.95 45.72) (width 0.25) (layer F.Cu) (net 3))
 (segment (start 107.95 48.92) (end 107.95 55.22) (width 0.25) (layer F.Cu) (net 3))
 (segment (start 59.69 40.64) (end 59.69 33.02) (width 0.25) (layer F.Cu) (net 4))
 (segment (start 59.69 30.48) (end 59.69 33.02) (width 0.25) (layer F.Cu) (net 4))
 (segment (start 59.69 40.64) (end 59.69 54.61) (width 0.25) (layer F.Cu) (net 4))
 (segment (start 59.69 54.61) (end 65.38 54.61) (width 0.25) (layer F.Cu) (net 4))
 (segment (start 59.08 67.725) (end 61.205 69.85) (width 0.25) (layer F.Cu) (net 4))
 (segment (start 59.08 54.61) (end 59.08 67.725) (width 0.25) (layer F.Cu) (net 4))
 (segment (start 96.52 69.85) (end 63.255 69.85) (width 0.25) (layer F.Cu) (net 5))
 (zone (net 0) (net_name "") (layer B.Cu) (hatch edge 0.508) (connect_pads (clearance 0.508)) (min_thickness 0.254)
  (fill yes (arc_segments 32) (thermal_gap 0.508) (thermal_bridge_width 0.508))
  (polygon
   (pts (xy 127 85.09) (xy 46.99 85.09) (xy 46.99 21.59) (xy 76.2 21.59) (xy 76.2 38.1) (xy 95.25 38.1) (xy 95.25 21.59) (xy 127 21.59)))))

